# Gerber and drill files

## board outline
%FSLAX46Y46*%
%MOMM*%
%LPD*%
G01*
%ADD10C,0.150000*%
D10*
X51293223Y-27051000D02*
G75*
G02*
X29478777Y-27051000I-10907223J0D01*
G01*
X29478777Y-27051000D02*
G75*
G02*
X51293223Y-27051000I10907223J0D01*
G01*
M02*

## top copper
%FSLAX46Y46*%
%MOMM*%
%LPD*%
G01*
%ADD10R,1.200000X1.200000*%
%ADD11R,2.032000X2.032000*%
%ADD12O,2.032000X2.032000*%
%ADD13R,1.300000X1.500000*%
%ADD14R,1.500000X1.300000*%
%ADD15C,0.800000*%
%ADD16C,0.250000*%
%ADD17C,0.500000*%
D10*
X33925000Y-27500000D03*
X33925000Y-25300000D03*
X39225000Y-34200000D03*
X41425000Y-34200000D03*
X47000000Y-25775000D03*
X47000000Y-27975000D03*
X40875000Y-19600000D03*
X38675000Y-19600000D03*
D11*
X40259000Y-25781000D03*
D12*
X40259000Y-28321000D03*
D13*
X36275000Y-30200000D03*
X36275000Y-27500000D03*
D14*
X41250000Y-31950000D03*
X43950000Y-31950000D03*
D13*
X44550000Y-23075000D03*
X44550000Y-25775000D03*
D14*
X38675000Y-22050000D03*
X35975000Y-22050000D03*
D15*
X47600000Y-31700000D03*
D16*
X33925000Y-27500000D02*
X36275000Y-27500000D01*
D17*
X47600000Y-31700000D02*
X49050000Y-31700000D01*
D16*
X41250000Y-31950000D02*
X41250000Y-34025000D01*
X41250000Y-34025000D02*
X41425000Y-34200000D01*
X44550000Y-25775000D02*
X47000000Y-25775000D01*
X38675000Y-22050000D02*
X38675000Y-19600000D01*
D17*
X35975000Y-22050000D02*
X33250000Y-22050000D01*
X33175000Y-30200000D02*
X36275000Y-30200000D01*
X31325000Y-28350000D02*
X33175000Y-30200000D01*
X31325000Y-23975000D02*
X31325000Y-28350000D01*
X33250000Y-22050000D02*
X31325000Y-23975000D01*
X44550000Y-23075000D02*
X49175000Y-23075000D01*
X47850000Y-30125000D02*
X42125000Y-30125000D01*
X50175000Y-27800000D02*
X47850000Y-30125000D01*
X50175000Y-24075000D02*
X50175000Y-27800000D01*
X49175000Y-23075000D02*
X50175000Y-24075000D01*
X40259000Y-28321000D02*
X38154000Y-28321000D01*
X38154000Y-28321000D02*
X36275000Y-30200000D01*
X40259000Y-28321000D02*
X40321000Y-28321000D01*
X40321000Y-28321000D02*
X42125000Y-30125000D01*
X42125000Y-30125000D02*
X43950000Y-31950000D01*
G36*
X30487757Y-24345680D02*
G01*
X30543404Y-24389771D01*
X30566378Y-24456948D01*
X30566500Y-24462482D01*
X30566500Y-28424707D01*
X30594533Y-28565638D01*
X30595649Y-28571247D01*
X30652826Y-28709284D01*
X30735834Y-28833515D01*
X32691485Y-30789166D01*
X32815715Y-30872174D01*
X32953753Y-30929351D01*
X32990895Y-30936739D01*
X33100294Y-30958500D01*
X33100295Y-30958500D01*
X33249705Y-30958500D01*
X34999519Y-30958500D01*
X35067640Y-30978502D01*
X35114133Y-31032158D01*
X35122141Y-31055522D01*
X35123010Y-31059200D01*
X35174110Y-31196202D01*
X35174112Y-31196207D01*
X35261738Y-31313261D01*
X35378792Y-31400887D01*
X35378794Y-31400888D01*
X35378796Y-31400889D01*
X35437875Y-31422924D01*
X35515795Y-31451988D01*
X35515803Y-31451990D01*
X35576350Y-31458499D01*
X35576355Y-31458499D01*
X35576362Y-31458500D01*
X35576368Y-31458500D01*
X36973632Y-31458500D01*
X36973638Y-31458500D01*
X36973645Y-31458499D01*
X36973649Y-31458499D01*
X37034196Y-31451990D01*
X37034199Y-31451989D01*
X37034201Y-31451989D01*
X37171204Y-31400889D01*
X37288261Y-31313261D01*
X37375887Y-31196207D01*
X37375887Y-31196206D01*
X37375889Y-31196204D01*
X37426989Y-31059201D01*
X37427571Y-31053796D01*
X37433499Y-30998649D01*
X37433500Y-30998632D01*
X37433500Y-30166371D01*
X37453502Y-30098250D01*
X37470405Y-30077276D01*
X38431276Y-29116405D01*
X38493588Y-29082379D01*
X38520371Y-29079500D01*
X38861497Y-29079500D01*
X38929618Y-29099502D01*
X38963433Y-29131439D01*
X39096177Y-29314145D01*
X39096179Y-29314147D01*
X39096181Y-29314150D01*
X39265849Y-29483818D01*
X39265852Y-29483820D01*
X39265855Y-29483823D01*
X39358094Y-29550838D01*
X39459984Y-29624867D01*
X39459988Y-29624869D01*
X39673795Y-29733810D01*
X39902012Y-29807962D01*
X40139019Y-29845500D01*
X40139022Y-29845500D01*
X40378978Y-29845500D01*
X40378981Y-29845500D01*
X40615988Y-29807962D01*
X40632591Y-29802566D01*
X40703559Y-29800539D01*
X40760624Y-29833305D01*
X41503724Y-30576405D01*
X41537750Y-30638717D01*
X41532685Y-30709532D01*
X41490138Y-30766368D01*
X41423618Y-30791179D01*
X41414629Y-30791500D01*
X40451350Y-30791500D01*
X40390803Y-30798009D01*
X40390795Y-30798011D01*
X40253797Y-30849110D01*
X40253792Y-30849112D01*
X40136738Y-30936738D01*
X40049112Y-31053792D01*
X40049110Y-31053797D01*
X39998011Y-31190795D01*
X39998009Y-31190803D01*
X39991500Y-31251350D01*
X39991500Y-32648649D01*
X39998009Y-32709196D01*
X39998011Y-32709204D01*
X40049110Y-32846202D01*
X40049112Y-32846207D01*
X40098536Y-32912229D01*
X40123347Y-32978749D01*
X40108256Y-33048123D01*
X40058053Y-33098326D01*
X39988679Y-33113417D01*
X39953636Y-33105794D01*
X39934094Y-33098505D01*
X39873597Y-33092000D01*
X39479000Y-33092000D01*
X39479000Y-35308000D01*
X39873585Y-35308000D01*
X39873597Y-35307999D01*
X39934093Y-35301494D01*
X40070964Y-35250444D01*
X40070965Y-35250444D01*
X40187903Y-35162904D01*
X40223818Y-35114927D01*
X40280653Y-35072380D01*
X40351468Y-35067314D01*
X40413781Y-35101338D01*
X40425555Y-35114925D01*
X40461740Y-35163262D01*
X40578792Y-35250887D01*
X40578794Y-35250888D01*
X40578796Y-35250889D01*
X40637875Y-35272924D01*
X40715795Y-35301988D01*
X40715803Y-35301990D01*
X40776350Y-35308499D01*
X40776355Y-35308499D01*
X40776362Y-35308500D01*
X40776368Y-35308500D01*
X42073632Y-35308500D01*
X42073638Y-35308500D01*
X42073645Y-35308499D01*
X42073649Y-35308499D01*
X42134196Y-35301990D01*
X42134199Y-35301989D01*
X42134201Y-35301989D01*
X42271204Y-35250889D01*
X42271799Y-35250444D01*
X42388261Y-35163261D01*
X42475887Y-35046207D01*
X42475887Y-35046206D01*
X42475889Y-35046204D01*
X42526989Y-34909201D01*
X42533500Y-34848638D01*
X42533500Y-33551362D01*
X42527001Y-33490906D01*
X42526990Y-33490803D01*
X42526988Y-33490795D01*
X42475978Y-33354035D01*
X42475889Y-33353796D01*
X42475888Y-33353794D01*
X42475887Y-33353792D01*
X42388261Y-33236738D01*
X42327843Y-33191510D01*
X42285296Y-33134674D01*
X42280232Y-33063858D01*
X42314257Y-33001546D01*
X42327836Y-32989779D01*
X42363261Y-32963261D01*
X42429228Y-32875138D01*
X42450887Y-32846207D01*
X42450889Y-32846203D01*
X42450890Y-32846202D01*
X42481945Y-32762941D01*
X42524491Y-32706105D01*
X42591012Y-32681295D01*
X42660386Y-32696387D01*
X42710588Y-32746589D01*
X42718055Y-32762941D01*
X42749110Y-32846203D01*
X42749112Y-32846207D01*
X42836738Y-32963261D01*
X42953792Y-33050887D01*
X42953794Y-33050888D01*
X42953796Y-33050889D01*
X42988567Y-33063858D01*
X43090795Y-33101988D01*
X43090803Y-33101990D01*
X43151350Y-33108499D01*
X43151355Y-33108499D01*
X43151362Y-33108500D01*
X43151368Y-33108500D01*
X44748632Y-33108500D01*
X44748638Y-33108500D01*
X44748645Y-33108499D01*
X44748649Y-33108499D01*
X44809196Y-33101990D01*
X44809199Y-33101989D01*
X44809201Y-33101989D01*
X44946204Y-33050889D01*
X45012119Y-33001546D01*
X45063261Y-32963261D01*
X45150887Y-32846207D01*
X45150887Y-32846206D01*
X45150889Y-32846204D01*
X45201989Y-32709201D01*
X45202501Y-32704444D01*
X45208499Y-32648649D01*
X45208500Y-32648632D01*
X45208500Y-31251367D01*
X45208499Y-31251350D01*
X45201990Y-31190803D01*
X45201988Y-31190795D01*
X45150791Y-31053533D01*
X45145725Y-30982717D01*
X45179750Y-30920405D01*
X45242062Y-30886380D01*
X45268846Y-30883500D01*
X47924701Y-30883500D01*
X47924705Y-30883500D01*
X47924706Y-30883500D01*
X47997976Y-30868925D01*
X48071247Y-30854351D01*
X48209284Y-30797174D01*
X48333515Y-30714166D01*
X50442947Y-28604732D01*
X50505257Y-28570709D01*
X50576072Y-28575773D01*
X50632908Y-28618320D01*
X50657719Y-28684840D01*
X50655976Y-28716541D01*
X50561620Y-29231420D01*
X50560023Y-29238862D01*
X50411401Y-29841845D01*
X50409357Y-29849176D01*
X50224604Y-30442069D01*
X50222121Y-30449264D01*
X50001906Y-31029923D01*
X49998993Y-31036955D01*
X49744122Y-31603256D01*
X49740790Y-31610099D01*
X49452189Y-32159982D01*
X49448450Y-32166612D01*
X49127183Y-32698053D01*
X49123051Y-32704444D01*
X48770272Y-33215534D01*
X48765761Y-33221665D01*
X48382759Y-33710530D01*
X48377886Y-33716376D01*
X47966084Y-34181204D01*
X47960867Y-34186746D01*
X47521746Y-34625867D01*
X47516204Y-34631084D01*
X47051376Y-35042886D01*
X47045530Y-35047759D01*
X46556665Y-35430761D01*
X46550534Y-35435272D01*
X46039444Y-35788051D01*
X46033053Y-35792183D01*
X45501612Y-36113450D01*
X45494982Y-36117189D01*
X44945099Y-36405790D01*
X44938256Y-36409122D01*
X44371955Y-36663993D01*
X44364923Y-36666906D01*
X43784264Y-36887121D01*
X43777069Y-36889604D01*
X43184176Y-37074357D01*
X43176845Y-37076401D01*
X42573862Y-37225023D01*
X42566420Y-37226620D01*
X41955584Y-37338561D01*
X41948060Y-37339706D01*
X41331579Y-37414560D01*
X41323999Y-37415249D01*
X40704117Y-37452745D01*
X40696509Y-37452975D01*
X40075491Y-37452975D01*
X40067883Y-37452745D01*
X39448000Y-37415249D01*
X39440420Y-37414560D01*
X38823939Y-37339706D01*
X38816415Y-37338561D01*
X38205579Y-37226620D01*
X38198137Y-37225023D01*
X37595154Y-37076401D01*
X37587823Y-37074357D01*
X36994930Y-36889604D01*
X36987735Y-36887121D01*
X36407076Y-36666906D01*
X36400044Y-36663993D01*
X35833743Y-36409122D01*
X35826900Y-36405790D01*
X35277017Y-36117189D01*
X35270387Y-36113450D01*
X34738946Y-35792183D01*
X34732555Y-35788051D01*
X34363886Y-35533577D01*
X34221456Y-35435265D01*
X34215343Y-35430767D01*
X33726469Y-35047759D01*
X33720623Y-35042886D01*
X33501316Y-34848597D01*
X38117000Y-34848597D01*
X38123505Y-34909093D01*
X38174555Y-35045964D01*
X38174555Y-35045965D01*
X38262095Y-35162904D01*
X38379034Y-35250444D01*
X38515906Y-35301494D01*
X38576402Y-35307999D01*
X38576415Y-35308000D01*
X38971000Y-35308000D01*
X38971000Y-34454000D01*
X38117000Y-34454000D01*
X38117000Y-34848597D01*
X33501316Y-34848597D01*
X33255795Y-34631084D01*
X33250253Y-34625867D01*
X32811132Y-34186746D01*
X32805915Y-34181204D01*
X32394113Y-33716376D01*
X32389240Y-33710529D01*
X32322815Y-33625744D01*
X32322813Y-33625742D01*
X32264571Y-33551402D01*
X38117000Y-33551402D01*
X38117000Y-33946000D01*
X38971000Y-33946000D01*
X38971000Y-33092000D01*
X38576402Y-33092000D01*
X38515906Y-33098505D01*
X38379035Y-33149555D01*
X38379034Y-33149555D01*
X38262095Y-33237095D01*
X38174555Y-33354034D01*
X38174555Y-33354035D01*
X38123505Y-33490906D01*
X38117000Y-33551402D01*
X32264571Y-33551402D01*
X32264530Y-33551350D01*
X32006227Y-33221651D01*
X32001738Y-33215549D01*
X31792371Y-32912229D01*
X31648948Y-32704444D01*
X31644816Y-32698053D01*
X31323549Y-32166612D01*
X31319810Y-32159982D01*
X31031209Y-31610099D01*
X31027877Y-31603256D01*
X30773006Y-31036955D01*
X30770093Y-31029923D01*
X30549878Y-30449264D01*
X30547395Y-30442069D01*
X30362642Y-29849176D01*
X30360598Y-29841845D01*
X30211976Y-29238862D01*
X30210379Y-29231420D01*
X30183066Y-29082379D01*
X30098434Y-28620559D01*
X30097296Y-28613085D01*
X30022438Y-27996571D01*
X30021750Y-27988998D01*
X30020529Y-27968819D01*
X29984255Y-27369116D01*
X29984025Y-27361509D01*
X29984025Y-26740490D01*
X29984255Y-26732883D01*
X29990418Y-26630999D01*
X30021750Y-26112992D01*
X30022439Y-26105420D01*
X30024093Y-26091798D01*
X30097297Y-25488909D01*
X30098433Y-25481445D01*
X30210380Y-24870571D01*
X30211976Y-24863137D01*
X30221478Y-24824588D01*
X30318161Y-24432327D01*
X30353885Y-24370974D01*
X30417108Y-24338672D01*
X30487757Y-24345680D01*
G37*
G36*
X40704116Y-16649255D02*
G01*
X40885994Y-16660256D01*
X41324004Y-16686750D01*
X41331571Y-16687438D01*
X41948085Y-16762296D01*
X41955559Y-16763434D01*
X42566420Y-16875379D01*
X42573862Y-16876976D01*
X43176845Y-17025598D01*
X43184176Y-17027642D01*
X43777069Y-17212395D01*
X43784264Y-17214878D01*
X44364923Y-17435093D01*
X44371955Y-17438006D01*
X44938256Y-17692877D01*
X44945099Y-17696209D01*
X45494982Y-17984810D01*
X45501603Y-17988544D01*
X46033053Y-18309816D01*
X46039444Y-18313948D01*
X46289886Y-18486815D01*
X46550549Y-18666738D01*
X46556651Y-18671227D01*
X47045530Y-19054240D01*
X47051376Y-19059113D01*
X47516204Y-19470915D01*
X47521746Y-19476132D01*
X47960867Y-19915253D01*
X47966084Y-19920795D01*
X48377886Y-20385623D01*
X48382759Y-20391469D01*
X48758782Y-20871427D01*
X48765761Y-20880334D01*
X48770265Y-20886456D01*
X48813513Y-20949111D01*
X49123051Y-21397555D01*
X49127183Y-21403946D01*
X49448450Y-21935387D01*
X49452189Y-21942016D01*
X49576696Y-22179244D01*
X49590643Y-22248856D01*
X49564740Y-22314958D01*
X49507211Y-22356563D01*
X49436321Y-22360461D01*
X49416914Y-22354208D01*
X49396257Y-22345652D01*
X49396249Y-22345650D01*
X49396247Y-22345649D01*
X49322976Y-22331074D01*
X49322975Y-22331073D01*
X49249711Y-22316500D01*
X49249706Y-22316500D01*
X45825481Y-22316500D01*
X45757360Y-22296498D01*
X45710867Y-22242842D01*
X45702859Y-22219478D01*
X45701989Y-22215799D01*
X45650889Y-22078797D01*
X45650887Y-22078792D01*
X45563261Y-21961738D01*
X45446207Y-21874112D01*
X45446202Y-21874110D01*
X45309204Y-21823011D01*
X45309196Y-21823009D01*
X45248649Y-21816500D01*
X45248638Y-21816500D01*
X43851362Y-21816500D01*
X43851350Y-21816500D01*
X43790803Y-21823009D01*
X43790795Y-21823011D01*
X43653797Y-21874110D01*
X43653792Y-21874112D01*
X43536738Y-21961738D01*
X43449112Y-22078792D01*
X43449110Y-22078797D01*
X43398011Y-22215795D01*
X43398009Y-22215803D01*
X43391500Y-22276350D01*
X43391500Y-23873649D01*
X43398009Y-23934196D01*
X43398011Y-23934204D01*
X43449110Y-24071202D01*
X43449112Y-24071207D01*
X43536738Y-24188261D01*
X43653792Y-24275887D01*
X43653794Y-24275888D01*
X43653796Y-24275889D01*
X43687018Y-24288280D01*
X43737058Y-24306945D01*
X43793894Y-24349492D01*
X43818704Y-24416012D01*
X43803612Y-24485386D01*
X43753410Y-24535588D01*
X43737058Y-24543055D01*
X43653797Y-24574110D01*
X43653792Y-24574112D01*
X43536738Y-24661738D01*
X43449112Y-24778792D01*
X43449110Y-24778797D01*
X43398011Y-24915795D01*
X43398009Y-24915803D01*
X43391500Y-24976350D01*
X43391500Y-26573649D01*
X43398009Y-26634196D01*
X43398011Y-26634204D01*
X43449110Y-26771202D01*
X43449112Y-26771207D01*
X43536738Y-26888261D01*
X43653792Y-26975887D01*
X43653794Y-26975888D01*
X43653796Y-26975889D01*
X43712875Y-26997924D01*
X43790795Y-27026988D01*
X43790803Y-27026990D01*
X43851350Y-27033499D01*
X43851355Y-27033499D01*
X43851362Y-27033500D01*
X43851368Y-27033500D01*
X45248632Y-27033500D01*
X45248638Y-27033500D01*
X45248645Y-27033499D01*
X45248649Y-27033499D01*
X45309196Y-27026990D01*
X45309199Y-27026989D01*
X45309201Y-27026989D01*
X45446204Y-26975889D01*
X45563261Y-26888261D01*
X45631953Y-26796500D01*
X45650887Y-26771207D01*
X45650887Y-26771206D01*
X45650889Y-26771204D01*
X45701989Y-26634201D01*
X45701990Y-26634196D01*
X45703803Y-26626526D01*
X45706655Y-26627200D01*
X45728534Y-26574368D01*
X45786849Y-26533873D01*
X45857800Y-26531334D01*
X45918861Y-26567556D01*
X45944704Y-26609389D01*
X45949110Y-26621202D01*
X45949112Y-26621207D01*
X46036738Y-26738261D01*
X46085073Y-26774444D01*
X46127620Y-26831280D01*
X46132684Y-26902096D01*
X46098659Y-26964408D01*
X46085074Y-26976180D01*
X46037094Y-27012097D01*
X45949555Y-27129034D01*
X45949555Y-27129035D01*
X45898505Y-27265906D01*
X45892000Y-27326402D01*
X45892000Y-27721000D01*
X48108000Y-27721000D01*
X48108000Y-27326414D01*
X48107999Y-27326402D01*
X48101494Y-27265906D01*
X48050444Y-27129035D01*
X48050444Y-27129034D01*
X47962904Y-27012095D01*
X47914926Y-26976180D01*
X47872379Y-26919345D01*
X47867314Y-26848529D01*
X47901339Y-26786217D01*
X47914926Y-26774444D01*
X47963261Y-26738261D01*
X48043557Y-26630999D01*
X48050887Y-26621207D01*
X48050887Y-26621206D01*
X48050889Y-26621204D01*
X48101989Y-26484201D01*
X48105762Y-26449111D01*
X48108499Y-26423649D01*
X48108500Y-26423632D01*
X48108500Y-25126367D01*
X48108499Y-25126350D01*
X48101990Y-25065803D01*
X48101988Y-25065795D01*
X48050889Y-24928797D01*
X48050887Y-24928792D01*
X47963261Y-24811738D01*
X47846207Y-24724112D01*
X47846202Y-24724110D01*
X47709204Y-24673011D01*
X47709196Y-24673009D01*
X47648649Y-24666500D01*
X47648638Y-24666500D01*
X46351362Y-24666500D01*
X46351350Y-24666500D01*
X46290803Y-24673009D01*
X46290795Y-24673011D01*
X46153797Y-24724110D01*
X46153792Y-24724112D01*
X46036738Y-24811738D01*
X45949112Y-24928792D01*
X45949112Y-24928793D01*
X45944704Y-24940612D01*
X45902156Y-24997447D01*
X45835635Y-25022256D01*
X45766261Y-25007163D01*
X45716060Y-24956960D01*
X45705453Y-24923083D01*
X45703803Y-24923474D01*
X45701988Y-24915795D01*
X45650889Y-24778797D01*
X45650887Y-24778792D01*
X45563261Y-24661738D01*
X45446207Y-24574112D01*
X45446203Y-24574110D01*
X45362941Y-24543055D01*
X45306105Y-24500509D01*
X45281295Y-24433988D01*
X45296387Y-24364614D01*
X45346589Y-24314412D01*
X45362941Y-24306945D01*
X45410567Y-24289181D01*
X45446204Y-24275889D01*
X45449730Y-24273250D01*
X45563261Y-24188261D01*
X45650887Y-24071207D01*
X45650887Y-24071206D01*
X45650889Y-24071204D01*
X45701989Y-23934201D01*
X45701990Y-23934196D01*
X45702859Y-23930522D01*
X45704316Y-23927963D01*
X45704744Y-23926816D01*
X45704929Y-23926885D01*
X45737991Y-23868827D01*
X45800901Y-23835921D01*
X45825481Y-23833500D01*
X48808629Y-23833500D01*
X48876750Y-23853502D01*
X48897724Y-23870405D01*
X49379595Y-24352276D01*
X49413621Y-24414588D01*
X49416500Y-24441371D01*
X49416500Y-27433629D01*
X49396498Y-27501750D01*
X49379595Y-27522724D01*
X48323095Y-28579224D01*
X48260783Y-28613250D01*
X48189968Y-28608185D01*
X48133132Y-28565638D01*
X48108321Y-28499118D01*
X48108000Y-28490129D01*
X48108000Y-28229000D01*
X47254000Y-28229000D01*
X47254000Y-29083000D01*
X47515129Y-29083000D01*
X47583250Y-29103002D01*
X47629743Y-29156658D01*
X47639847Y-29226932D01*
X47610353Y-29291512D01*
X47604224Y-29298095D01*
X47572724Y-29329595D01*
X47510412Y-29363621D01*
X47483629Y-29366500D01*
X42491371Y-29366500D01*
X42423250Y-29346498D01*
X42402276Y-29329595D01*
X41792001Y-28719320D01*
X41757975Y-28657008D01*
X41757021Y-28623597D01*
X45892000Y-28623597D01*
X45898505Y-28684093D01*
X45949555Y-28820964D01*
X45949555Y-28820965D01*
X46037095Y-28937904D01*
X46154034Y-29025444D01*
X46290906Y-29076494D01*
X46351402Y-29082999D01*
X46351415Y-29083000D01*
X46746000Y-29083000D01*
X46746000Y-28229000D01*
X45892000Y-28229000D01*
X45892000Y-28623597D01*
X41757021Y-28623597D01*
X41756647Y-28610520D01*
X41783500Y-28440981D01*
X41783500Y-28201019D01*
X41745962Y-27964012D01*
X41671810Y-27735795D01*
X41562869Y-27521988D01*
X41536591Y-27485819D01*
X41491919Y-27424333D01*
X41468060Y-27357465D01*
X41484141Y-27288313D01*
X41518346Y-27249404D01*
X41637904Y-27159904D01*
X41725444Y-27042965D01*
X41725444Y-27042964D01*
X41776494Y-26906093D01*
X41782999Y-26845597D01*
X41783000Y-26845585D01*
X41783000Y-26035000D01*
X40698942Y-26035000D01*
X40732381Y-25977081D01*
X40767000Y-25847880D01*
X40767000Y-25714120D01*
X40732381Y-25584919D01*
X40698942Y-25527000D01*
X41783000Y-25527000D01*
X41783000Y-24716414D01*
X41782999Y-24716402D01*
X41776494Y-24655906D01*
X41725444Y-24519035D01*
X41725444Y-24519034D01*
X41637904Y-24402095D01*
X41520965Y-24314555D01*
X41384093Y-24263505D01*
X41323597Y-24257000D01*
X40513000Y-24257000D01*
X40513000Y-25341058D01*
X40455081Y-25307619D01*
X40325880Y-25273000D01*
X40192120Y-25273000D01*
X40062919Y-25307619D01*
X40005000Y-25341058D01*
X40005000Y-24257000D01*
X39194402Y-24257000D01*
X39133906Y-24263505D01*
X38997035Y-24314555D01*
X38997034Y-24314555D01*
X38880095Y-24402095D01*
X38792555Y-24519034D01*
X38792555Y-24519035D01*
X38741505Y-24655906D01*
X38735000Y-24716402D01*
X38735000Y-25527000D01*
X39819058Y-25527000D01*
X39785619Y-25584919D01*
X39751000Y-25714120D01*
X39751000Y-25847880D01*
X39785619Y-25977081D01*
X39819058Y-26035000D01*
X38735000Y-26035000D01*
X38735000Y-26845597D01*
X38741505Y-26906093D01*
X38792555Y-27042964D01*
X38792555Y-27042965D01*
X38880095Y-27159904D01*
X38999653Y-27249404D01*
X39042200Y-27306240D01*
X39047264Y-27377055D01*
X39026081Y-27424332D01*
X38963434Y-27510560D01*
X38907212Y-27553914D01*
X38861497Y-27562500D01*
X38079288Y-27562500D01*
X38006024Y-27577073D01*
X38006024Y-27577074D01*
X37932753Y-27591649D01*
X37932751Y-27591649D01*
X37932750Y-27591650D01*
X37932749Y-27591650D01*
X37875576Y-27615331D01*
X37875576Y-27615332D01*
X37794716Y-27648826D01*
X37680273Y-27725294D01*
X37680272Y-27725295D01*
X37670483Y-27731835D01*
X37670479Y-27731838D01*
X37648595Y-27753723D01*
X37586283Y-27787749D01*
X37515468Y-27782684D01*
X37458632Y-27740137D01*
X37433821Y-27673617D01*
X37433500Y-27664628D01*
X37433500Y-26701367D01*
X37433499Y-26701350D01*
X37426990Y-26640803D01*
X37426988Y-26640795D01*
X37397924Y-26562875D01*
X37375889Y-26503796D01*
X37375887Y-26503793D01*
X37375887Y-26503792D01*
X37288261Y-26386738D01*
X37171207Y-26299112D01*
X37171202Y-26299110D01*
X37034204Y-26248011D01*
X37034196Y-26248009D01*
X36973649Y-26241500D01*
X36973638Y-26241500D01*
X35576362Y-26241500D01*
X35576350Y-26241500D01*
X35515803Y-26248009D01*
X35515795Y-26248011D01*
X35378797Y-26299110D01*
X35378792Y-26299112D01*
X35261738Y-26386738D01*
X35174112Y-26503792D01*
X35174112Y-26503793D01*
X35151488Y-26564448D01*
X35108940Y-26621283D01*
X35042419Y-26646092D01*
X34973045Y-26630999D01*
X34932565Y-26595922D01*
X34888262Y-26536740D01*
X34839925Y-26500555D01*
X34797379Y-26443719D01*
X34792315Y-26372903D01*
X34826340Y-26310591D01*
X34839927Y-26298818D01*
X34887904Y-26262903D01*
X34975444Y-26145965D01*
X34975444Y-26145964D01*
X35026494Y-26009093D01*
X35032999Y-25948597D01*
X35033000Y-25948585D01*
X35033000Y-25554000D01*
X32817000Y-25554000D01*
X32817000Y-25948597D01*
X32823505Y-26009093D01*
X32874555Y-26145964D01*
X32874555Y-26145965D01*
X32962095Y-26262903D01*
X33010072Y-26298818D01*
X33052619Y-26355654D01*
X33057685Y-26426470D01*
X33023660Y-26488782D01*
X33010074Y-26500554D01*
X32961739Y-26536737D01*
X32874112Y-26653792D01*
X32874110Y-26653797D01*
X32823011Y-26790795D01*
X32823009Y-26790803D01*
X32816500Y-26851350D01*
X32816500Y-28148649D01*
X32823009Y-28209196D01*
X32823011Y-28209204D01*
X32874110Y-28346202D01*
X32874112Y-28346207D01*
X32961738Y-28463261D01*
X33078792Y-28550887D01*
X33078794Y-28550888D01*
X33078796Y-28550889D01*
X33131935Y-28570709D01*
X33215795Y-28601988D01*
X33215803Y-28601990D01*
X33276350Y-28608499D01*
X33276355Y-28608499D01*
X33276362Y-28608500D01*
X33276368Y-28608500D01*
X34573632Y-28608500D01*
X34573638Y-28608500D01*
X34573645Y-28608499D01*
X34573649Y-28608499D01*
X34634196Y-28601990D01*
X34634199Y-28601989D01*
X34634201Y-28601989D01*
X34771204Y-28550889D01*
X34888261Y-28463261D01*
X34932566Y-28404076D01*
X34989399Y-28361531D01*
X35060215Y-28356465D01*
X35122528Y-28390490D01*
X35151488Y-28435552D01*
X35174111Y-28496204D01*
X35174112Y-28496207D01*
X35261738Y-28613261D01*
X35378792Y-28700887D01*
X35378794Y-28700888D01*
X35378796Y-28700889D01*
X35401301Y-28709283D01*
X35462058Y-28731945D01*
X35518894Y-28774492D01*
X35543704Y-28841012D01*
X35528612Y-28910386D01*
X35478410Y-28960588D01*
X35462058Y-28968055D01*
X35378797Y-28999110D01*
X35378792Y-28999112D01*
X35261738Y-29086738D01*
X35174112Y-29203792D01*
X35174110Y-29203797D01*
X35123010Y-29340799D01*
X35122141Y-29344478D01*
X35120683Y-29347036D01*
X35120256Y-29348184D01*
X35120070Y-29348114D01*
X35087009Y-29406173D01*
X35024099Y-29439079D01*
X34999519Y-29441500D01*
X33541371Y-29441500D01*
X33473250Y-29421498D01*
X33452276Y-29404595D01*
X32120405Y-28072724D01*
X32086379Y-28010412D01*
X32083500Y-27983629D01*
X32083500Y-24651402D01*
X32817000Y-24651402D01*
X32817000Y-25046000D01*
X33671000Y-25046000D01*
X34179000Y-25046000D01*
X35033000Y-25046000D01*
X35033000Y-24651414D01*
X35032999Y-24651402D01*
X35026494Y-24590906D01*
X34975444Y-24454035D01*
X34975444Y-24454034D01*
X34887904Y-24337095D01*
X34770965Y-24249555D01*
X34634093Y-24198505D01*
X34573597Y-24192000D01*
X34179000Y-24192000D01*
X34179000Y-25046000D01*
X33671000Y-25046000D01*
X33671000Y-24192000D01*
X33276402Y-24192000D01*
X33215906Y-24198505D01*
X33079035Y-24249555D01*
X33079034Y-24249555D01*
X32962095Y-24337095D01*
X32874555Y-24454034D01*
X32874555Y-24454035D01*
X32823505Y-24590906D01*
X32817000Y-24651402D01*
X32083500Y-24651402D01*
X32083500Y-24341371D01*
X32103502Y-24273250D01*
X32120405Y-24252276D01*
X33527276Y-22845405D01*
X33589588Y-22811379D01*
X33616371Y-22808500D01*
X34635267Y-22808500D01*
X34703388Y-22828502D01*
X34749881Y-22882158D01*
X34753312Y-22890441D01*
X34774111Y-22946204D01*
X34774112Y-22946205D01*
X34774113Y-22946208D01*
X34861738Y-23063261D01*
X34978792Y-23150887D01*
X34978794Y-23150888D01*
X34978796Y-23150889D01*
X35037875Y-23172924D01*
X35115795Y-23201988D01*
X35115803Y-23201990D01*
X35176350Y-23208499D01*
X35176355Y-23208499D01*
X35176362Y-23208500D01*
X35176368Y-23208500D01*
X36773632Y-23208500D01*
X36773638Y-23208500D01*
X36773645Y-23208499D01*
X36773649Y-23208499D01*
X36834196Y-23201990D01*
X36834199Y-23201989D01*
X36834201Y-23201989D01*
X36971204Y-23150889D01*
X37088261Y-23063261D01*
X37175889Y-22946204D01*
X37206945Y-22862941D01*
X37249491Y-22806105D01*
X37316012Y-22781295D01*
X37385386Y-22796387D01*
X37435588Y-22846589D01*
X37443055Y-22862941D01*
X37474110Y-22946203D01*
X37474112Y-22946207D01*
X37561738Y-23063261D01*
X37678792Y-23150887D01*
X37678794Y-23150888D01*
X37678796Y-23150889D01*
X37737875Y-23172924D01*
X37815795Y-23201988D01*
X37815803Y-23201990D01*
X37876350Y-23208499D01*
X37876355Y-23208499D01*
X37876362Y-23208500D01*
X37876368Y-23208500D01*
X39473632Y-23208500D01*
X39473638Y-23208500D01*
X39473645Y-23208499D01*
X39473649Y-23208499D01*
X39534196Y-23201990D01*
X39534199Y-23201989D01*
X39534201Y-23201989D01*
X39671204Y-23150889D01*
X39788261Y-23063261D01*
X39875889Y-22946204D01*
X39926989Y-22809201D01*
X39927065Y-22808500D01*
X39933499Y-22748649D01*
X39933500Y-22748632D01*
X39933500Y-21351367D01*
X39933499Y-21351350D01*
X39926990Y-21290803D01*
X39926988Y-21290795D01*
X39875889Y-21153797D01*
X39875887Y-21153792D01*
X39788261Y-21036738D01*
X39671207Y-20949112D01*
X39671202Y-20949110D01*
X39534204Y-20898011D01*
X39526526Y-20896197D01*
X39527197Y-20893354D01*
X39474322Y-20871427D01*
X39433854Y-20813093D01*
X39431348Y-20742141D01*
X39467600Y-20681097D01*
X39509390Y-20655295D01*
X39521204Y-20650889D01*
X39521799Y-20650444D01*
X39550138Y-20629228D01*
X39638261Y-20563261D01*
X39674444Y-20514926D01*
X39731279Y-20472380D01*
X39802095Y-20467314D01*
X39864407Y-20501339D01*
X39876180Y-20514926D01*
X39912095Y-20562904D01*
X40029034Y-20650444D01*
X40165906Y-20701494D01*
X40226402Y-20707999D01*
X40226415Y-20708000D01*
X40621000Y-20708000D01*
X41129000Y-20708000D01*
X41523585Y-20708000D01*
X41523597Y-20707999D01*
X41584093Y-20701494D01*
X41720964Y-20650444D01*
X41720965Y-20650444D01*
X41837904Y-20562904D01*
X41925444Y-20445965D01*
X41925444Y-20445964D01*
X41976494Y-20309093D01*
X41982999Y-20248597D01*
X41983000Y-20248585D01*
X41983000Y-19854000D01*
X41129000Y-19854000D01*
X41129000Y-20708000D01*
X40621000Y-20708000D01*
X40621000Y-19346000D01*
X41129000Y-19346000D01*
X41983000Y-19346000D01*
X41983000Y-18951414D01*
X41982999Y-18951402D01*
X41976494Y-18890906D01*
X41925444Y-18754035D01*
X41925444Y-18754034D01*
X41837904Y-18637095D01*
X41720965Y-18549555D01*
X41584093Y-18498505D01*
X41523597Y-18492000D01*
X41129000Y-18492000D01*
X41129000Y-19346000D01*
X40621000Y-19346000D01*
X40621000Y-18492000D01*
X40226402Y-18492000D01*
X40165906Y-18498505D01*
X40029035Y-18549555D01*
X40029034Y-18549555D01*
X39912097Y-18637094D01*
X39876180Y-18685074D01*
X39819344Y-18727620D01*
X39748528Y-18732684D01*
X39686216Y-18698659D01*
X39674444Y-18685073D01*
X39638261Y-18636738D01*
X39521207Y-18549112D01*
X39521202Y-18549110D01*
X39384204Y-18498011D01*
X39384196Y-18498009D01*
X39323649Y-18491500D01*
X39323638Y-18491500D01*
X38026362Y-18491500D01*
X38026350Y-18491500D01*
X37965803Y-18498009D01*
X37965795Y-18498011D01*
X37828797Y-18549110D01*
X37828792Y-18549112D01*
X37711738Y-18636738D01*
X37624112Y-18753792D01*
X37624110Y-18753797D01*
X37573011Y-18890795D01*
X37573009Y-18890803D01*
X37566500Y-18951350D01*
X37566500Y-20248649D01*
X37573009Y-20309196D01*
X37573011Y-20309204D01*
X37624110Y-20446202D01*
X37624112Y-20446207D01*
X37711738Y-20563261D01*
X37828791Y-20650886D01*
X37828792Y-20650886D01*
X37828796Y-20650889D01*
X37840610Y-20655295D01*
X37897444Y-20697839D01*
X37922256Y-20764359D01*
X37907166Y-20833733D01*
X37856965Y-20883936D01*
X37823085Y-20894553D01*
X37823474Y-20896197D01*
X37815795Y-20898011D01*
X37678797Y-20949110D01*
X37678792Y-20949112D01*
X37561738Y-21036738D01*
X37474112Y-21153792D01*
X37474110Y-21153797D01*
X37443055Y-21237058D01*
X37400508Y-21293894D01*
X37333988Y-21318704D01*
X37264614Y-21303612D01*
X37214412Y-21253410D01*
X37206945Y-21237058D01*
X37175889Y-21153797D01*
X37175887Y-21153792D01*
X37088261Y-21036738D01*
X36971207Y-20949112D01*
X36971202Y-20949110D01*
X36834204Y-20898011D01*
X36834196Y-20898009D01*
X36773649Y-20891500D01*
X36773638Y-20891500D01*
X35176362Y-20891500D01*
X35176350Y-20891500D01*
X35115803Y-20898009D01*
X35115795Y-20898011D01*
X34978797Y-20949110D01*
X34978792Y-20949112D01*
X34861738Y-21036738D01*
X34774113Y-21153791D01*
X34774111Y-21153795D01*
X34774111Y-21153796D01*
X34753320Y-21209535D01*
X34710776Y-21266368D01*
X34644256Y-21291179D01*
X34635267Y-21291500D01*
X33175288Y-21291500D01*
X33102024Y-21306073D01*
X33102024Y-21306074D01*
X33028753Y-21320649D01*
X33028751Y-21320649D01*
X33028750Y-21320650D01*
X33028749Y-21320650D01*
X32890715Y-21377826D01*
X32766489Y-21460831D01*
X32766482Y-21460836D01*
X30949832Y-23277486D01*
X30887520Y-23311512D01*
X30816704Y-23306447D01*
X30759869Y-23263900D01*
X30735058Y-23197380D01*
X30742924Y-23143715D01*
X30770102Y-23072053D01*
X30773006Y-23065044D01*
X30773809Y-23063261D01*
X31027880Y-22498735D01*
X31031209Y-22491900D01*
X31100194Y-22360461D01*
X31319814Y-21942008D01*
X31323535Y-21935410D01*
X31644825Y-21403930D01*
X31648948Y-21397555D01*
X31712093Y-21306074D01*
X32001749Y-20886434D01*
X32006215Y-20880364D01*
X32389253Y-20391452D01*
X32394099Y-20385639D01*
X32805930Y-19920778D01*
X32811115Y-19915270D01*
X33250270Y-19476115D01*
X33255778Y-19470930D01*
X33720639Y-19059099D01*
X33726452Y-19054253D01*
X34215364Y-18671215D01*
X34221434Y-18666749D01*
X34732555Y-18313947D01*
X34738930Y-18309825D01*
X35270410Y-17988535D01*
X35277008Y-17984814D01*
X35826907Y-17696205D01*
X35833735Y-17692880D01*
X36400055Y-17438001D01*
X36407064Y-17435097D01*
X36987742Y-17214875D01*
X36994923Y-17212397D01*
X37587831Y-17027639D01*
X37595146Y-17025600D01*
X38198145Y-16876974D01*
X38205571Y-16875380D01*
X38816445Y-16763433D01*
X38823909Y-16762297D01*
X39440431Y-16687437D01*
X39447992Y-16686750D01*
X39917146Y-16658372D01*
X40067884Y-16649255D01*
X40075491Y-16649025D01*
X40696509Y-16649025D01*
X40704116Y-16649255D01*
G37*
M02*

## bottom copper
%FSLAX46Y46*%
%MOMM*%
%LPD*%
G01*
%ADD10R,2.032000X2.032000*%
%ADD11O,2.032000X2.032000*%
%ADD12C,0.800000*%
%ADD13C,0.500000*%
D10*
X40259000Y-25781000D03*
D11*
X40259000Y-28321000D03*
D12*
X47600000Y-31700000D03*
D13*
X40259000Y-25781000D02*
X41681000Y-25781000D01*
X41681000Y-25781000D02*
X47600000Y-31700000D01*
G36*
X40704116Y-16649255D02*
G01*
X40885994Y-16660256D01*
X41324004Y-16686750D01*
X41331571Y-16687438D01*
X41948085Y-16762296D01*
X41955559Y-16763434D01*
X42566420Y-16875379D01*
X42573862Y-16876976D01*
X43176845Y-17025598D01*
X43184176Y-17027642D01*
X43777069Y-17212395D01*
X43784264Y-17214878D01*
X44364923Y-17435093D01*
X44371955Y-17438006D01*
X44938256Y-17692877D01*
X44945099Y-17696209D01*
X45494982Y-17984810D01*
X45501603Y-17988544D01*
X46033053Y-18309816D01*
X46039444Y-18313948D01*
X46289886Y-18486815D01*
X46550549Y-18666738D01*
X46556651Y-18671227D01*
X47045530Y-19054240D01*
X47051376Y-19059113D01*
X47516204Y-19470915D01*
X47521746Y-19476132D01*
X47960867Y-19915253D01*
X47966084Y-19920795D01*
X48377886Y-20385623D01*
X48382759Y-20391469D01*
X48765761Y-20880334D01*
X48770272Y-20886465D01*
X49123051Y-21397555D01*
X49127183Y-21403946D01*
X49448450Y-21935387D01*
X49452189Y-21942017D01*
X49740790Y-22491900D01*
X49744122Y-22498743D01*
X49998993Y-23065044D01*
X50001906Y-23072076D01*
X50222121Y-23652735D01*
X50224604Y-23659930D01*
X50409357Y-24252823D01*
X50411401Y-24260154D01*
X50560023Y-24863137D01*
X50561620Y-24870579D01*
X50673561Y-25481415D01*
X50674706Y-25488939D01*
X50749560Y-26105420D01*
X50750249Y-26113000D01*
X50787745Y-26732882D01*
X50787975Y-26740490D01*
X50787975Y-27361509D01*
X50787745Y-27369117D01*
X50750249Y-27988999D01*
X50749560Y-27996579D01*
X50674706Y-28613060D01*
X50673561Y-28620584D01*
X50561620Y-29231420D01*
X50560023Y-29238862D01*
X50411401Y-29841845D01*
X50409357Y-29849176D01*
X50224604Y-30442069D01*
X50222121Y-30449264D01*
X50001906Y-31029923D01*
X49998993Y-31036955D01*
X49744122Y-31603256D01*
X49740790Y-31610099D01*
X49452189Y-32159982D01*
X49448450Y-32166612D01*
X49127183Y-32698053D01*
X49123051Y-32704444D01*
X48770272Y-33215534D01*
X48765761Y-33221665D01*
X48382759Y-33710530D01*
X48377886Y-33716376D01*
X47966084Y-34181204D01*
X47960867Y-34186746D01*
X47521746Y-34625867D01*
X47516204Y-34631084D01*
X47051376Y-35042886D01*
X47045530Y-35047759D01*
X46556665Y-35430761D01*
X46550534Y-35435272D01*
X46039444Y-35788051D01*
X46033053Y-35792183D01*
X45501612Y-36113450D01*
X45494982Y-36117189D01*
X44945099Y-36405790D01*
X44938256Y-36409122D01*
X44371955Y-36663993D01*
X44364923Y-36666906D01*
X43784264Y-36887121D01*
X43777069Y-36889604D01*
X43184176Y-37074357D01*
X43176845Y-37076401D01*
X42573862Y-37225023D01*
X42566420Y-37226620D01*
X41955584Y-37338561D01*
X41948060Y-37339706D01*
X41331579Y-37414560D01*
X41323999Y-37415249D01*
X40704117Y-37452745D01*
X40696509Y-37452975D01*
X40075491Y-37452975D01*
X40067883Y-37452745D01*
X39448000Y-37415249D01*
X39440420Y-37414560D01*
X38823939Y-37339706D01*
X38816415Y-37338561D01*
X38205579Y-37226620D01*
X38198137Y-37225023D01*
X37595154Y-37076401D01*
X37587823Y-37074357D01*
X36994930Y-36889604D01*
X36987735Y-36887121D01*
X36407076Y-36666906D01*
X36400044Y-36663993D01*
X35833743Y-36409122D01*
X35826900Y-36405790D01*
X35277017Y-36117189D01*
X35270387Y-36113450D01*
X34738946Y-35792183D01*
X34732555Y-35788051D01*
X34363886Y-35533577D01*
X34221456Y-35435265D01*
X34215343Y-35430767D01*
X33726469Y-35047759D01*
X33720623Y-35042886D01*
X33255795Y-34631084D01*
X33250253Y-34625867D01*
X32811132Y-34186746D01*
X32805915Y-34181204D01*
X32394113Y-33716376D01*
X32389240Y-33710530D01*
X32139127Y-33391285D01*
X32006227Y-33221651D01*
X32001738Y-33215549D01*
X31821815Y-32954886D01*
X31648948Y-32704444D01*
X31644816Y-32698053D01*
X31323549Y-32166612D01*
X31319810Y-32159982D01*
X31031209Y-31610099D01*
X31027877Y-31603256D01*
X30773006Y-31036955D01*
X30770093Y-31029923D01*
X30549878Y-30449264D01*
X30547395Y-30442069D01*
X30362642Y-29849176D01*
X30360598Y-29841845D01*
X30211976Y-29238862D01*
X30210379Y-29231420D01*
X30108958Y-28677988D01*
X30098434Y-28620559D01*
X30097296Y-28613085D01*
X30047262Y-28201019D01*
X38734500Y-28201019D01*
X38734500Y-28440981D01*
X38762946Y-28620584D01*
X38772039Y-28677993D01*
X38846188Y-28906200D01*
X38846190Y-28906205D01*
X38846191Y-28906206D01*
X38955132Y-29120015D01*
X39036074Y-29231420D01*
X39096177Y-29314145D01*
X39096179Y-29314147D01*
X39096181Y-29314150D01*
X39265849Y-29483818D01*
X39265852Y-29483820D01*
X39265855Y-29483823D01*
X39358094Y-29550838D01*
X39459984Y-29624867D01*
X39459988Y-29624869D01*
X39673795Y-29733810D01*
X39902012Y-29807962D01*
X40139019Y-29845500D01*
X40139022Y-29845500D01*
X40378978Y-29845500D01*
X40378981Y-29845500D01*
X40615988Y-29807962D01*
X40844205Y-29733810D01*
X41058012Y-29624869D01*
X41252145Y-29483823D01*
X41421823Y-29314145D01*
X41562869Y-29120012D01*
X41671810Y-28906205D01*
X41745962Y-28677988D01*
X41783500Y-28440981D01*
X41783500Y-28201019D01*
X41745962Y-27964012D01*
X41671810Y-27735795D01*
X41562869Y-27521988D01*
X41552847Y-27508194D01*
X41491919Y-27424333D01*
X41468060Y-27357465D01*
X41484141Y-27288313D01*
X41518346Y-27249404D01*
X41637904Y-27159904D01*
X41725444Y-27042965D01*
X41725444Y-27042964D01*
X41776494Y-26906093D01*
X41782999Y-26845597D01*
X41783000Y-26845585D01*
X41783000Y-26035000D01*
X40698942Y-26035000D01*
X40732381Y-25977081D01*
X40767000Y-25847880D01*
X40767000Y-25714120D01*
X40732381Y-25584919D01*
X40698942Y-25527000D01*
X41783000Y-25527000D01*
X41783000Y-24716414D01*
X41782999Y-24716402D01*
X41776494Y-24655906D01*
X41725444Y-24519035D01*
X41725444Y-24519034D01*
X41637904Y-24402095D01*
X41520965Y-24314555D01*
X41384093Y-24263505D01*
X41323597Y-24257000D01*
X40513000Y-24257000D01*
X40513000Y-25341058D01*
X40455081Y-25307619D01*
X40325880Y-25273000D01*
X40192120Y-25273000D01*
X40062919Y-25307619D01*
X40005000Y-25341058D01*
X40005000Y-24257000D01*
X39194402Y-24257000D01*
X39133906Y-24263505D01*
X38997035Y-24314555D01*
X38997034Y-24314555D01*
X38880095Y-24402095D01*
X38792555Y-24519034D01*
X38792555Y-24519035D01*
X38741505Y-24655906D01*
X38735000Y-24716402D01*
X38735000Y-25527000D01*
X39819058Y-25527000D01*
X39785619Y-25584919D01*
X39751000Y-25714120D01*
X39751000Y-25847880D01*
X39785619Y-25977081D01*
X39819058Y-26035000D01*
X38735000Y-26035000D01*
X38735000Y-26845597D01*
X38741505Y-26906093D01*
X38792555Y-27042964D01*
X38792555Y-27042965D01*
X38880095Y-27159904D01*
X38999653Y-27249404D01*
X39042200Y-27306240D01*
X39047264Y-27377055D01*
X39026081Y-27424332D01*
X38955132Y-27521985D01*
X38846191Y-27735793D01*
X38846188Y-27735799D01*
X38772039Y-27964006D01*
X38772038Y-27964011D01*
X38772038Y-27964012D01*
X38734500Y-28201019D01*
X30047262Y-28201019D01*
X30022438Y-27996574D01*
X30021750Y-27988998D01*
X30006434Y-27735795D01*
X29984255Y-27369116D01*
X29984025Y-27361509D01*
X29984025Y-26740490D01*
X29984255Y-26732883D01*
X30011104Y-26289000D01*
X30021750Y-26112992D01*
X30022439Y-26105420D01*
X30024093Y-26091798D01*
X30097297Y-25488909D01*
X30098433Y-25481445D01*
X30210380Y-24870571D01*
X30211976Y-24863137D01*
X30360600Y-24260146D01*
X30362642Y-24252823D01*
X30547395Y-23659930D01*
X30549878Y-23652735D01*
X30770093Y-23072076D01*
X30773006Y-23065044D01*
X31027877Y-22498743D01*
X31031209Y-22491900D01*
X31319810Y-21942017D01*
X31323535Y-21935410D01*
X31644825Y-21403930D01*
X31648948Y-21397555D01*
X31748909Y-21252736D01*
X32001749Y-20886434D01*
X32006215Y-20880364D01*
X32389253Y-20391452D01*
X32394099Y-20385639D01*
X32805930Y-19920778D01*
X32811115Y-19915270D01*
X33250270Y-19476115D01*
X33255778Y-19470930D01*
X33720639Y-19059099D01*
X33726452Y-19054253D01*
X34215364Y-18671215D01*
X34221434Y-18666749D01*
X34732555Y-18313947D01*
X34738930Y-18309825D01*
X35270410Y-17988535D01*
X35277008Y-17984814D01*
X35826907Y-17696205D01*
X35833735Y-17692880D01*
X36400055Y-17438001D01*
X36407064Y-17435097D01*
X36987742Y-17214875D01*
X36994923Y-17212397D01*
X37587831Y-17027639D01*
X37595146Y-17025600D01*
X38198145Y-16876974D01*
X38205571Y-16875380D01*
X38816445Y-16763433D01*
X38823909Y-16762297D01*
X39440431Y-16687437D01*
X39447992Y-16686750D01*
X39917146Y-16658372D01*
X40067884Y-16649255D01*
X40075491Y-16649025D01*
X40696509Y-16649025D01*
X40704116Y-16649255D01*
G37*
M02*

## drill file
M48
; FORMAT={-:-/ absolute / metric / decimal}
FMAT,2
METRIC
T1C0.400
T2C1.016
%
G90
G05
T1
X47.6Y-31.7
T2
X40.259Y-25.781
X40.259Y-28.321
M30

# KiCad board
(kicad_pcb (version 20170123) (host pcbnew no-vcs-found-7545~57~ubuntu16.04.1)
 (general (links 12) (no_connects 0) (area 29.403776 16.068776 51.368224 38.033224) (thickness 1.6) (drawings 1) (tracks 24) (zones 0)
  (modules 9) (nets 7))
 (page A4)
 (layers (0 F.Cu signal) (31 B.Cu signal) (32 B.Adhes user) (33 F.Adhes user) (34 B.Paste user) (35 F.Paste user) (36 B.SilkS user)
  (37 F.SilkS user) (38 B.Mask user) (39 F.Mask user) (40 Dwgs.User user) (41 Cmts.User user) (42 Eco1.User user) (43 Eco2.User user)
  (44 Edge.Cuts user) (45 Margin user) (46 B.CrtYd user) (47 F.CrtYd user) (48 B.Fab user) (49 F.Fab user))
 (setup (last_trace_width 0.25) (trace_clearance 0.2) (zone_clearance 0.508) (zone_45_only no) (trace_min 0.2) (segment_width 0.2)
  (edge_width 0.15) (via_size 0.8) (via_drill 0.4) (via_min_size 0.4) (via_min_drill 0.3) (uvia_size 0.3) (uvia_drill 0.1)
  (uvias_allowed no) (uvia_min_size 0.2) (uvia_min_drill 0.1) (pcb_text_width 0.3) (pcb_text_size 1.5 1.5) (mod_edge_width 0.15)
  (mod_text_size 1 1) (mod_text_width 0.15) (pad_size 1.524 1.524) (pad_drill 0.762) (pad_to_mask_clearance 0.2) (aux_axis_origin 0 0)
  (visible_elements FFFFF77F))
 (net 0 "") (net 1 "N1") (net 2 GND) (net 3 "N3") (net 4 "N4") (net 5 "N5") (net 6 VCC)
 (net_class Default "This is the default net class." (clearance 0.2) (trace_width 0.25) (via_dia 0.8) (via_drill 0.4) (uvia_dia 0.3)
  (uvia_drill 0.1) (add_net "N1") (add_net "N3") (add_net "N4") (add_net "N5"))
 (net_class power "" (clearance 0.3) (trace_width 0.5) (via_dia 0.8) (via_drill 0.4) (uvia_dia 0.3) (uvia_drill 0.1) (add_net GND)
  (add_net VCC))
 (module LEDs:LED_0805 (layer F.Cu) (at 33.925 26.4 270)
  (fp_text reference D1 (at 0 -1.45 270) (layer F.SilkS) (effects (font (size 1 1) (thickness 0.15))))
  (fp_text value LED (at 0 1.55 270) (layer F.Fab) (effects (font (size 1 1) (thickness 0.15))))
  (pad 2 smd rect (at 1.1 0 90) (size 1.2 1.2) (layers F.Cu F.Paste F.Mask) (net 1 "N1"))
  (pad 1 smd rect (at -1.1 0 90) (size 1.2 1.2) (layers F.Cu F.Paste F.Mask) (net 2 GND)))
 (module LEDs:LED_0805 (layer F.Cu) (at 40.325 34.2)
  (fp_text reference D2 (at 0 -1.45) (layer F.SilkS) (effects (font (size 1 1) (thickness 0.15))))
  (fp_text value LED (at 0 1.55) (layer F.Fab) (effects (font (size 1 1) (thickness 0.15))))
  (pad 1 smd rect (at -1.1 0 180) (size 1.2 1.2) (layers F.Cu F.Paste F.Mask) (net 2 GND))
  (pad 2 smd rect (at 1.1 0 180) (size 1.2 1.2) (layers F.Cu F.Paste F.Mask) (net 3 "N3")))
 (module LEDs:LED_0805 (layer F.Cu) (at 47 26.875 90)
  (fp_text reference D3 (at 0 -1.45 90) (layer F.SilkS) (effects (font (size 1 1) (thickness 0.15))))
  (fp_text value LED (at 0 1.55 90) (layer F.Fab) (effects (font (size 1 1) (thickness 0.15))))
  (pad 2 smd rect (at 1.1 0 270) (size 1.2 1.2) (layers F.Cu F.Paste F.Mask) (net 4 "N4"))
  (pad 1 smd rect (at -1.1 0 270) (size 1.2 1.2) (layers F.Cu F.Paste F.Mask) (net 2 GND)))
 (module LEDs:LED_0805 (layer F.Cu) (at 39.775 19.6 180)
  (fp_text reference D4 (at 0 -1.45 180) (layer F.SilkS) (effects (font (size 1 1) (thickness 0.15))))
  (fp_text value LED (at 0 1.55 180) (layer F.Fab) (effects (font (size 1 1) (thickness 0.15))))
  (pad 1 smd rect (at -1.1 0) (size 1.2 1.2) (layers F.Cu F.Paste F.Mask) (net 2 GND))
  (pad 2 smd rect (at 1.1 0) (size 1.2 1.2) (layers F.Cu F.Paste F.Mask) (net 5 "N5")))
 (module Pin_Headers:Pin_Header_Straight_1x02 (layer F.Cu) (at 40.259 25.781)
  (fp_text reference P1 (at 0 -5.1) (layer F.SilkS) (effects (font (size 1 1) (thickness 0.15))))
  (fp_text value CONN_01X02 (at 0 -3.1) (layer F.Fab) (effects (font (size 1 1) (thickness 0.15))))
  (pad 1 thru_hole rect (at 0 0) (size 2.032 2.032) (drill 1.016) (layers *.Cu *.Mask F.SilkS) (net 2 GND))
  (pad 2 thru_hole oval (at 0 2.54) (size 2.032 2.032) (drill 1.016) (layers *.Cu *.Mask F.SilkS) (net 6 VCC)))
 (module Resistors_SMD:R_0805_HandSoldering (layer F.Cu) (at 36.275 28.85 90)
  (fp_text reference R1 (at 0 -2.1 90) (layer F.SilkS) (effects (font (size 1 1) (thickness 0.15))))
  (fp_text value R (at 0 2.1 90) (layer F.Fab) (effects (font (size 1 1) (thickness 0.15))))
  (pad 1 smd rect (at -1.35 0 90) (size 1.5 1.3) (layers F.Cu F.Paste F.Mask) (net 6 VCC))
  (pad 2 smd rect (at 1.35 0 90) (size 1.5 1.3) (layers F.Cu F.Paste F.Mask) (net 1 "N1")))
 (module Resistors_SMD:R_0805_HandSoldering (layer F.Cu) (at 42.6 31.95 180)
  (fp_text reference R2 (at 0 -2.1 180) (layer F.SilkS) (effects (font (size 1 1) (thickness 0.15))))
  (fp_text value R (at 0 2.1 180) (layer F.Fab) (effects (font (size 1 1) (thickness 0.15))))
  (pad 2 smd rect (at 1.35 0 180) (size 1.5 1.3) (layers F.Cu F.Paste F.Mask) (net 3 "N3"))
  (pad 1 smd rect (at -1.35 0 180) (size 1.5 1.3) (layers F.Cu F.Paste F.Mask) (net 6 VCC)))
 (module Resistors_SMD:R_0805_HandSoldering (layer F.Cu) (at 44.55 24.425 270)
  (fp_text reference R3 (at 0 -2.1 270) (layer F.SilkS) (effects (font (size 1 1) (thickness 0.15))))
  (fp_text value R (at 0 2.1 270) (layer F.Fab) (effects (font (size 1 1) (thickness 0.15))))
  (pad 1 smd rect (at -1.35 0 270) (size 1.5 1.3) (layers F.Cu F.Paste F.Mask) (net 6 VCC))
  (pad 2 smd rect (at 1.35 0 270) (size 1.5 1.3) (layers F.Cu F.Paste F.Mask) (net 4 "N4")))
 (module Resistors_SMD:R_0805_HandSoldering (layer F.Cu) (at 37.325 22.05)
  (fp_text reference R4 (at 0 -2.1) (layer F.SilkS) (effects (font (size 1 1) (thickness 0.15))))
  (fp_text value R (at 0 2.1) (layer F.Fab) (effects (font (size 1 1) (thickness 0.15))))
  (pad 2 smd rect (at 1.35 0) (size 1.5 1.3) (layers F.Cu F.Paste F.Mask) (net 5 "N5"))
  (pad 1 smd rect (at -1.35 0) (size 1.5 1.3) (layers F.Cu F.Paste F.Mask) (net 6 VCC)))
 (gr_circle (center 40.386 27.051) (end 35.306 17.399) (layer Edge.Cuts) (width 0.15))
 (segment (start 33.925 27.5) (end 36.275 27.5) (width 0.25) (layer F.Cu) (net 1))
 (segment (start 40.259 25.781) (end 41.681 25.781) (width 0.5) (layer B.Cu) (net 2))
 (segment (start 47.6 31.7) (end 49.05 31.7) (width 0.5) (layer F.Cu) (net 2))
 (via (at 47.6 31.7) (size 0.8) (drill 0.4) (layers F.Cu B.Cu) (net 2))
 (segment (start 41.681 25.781) (end 47.6 31.7) (width 0.5) (layer B.Cu) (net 2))
 (segment (start 41.25 31.95) (end 41.25 34.025) (width 0.25) (layer F.Cu) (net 3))
 (segment (start 41.25 34.025) (end 41.425 34.2) (width 0.25) (layer F.Cu) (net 3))
 (segment (start 44.55 25.775) (end 47 25.775) (width 0.25) (layer F.Cu) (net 4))
 (segment (start 38.675 22.05) (end 38.675 19.6) (width 0.25) (layer F.Cu) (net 5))
 (segment (start 35.975 22.05) (end 33.25 22.05) (width 0.5) (layer F.Cu) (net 6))
 (segment (start 33.175 30.2) (end 36.275 30.2) (width 0.5) (layer F.Cu) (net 6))
 (segment (start 31.325 28.35) (end 33.175 30.2) (width 0.5) (layer F.Cu) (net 6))
 (segment (start 31.325 23.975) (end 31.325 28.35) (width 0.5) (layer F.Cu) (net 6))
 (segment (start 33.25 22.05) (end 31.325 23.975) (width 0.5) (layer F.Cu) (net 6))
 (segment (start 44.55 23.075) (end 49.175 23.075) (width 0.5) (layer F.Cu) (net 6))
 (segment (start 47.85 30.125) (end 42.125 30.125) (width 0.5) (layer F.Cu) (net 6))
 (segment (start 50.175 27.8) (end 47.85 30.125) (width 0.5) (layer F.Cu) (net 6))
 (segment (start 50.175 24.075) (end 50.175 27.8) (width 0.5) (layer F.Cu) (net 6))
 (segment (start 49.175 23.075) (end 50.175 24.075) (width 0.5) (layer F.Cu) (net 6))
 (segment (start 40.259 28.321) (end 38.154 28.321) (width 0.5) (layer F.Cu) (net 6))
 (segment (start 38.154 28.321) (end 36.275 30.2) (width 0.5) (layer F.Cu) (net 6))
 (segment (start 40.259 28.321) (end 40.321 28.321) (width 0.5) (layer F.Cu) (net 6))
 (segment (start 40.321 28.321) (end 42.125 30.125) (width 0.5) (layer F.Cu) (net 6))
 (segment (start 42.125 30.125) (end 43.95 31.95) (width 0.5) (layer F.Cu) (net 6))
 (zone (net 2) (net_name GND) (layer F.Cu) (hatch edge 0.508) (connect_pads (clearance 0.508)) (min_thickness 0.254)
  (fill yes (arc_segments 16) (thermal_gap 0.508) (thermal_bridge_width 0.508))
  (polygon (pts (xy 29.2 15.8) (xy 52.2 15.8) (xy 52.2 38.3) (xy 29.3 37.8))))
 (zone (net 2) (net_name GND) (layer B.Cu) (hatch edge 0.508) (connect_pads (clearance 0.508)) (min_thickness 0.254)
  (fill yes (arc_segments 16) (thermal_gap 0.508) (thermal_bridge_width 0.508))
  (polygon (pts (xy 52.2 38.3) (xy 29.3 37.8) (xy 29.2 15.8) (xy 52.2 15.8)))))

